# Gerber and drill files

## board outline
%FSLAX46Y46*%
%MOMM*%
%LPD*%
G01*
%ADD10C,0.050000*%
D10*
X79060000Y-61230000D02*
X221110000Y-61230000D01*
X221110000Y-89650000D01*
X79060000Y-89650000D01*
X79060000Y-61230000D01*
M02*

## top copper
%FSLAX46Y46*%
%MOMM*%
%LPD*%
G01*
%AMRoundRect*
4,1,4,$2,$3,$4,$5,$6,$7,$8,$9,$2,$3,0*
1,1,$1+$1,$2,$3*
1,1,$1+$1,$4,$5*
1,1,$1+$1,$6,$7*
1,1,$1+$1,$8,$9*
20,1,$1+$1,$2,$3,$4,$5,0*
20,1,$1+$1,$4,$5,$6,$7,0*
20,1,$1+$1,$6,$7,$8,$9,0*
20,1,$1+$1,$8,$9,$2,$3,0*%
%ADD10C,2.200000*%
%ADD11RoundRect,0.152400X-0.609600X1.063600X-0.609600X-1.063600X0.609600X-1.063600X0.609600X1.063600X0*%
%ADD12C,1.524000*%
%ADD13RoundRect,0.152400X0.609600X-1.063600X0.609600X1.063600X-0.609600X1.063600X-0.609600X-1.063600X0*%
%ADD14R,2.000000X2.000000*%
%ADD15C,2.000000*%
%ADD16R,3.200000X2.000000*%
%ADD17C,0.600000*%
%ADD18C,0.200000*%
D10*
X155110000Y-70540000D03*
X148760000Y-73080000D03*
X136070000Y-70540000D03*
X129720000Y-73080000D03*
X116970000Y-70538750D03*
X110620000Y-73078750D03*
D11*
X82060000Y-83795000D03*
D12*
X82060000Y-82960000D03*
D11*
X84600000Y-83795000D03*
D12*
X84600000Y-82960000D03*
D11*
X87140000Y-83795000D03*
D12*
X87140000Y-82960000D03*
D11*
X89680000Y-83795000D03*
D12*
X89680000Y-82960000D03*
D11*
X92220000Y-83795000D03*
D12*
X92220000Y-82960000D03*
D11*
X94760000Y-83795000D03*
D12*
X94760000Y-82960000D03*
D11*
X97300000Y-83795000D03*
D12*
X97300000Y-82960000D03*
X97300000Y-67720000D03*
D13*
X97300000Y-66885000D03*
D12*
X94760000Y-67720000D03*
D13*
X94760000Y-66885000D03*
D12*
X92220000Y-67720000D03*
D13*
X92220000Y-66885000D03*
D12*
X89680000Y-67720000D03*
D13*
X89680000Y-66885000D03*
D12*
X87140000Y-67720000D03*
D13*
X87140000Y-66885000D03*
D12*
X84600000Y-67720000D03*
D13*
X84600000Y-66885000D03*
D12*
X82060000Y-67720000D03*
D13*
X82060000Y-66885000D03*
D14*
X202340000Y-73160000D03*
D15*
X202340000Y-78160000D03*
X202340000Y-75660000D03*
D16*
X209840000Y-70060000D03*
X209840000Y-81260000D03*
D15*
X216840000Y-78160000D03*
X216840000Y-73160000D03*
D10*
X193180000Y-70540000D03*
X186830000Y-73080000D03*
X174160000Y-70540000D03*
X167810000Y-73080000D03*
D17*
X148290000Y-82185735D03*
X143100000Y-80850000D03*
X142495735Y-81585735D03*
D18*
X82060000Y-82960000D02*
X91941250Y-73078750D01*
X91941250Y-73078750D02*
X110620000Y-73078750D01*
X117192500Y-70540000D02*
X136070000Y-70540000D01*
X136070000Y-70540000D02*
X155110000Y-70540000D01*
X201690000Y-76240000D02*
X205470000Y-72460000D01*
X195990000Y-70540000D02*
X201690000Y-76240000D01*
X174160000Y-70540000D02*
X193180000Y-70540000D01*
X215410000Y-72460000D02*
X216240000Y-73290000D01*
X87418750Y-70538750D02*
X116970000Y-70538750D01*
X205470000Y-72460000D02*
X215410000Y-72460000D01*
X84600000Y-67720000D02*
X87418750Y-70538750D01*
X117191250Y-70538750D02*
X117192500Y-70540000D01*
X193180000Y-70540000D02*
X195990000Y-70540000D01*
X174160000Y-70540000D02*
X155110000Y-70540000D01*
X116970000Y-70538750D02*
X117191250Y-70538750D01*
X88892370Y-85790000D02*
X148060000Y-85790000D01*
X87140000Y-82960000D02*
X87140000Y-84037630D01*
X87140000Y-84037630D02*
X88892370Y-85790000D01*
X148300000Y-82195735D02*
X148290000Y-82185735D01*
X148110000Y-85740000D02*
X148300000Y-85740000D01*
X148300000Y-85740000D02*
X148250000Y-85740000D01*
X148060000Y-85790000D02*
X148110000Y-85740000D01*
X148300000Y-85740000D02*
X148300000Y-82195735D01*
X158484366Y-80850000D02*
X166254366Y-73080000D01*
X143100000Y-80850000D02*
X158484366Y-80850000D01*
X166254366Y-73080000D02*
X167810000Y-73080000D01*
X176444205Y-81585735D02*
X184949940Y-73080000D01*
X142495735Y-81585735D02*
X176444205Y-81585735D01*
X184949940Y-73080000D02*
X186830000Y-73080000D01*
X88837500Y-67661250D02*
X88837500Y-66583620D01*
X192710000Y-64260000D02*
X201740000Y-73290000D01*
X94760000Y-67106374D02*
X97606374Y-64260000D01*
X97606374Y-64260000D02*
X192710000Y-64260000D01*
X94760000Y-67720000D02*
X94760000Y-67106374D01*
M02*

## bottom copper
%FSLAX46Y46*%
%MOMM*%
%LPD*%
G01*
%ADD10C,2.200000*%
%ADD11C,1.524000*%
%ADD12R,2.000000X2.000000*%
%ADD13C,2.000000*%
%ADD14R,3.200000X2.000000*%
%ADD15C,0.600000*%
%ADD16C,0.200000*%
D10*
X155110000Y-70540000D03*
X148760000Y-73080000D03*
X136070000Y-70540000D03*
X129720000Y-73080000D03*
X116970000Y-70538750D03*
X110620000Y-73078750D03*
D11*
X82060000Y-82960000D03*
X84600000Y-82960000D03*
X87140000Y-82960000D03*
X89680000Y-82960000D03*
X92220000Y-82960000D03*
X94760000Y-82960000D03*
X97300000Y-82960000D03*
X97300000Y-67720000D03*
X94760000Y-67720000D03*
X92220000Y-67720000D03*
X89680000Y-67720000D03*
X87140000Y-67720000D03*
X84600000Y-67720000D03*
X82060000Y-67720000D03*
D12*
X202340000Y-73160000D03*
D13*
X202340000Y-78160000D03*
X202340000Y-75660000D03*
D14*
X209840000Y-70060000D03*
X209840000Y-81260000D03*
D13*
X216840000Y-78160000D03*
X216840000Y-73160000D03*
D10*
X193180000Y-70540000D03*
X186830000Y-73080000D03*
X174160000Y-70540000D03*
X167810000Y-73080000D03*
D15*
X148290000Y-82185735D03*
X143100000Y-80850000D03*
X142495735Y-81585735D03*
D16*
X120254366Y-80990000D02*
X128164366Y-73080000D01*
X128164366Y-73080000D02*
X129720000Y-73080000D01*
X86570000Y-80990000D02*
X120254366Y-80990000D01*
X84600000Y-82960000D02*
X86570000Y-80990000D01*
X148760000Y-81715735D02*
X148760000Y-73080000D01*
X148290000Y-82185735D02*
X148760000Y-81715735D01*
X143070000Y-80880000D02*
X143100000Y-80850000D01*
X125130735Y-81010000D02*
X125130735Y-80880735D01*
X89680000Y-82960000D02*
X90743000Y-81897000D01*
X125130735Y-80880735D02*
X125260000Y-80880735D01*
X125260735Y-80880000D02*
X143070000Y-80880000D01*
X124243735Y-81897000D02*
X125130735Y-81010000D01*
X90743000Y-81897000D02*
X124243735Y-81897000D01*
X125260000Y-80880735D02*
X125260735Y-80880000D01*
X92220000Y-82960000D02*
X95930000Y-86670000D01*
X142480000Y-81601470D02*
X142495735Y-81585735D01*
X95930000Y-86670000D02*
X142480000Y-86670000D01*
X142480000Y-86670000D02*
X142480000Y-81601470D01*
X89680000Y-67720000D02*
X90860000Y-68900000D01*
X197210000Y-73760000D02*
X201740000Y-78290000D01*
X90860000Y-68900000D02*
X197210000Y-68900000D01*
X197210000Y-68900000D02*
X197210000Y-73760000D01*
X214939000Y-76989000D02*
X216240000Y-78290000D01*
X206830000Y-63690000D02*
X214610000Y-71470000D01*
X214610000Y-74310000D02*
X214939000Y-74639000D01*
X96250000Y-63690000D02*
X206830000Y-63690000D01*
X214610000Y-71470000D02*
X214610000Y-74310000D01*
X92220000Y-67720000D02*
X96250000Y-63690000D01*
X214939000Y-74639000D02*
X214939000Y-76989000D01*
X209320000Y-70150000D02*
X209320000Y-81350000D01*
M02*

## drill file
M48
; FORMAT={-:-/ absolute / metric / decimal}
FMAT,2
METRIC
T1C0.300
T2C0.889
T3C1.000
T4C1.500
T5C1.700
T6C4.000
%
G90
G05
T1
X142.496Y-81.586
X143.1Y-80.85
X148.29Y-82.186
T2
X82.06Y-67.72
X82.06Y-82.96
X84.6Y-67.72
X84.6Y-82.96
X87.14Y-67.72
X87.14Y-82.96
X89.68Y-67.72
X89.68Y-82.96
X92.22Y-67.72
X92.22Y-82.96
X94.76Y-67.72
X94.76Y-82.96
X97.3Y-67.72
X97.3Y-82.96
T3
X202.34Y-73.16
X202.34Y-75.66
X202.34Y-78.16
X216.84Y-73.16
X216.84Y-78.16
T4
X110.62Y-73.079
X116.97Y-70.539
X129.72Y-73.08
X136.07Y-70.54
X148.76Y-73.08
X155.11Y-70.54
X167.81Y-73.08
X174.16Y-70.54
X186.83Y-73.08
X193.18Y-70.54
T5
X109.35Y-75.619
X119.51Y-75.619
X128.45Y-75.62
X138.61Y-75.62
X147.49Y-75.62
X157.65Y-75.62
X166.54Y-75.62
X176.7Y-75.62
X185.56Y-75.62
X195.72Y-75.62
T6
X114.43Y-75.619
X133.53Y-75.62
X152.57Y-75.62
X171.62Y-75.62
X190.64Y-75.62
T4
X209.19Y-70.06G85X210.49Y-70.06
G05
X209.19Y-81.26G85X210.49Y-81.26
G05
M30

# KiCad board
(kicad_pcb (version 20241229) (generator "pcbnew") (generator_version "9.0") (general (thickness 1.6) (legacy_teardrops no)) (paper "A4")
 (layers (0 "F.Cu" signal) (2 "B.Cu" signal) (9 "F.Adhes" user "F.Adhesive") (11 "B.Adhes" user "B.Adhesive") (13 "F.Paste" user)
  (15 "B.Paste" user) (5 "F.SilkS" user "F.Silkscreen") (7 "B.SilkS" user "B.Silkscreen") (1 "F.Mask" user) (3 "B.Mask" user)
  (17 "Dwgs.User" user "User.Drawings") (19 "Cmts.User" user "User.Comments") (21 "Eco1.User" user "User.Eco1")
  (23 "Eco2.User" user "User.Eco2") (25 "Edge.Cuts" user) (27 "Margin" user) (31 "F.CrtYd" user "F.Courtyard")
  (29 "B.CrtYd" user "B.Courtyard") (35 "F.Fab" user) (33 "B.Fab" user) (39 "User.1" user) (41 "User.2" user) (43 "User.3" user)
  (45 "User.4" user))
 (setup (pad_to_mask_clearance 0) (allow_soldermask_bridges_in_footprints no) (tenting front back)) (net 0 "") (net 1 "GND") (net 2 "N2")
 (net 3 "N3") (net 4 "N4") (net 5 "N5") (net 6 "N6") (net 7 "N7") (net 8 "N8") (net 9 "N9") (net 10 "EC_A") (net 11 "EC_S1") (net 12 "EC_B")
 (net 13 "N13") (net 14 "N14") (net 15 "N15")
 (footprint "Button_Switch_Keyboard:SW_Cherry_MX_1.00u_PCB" (layer "F.Cu") (at 155.11 70.54)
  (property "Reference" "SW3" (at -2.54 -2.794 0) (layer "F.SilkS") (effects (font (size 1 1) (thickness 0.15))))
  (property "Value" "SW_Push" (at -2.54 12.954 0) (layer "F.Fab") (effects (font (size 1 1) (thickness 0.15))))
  (pad "" np_thru_hole circle (at -7.62 5.08) (size 1.7 1.7) (drill 1.7) (layers "*.Cu" "*.Mask"))
  (pad "" np_thru_hole circle (at -2.54 5.08) (size 4 4) (drill 4) (layers "*.Cu" "*.Mask"))
  (pad "" np_thru_hole circle (at 2.54 5.08) (size 1.7 1.7) (drill 1.7) (layers "*.Cu" "*.Mask"))
  (pad "1" thru_hole circle (at 0 0) (size 2.2 2.2) (drill 1.5) (layers "*.Cu" "*.Mask") (remove_unused_layers no) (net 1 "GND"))
  (pad "2" thru_hole circle (at -6.35 2.54) (size 2.2 2.2) (drill 1.5) (layers "*.Cu" "*.Mask") (remove_unused_layers no) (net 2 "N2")))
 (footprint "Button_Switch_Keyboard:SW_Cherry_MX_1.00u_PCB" (layer "F.Cu") (at 136.07 70.54)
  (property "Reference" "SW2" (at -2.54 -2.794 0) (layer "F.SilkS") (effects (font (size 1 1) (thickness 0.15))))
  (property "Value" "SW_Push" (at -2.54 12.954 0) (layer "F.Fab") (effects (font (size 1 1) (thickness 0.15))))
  (pad "" np_thru_hole circle (at -7.62 5.08) (size 1.7 1.7) (drill 1.7) (layers "*.Cu" "*.Mask"))
  (pad "" np_thru_hole circle (at -2.54 5.08) (size 4 4) (drill 4) (layers "*.Cu" "*.Mask"))
  (pad "" np_thru_hole circle (at 2.54 5.08) (size 1.7 1.7) (drill 1.7) (layers "*.Cu" "*.Mask"))
  (pad "1" thru_hole circle (at 0 0) (size 2.2 2.2) (drill 1.5) (layers "*.Cu" "*.Mask") (remove_unused_layers no) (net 1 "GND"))
  (pad "2" thru_hole circle (at -6.35 2.54) (size 2.2 2.2) (drill 1.5) (layers "*.Cu" "*.Mask") (remove_unused_layers no) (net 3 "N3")))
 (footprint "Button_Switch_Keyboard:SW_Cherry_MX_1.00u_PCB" (layer "F.Cu") (at 116.97 70.53875)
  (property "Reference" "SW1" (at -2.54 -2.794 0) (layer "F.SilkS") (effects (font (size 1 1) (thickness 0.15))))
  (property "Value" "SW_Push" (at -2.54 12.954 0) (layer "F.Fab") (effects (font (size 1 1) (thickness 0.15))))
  (pad "" np_thru_hole circle (at -7.62 5.08) (size 1.7 1.7) (drill 1.7) (layers "*.Cu" "*.Mask"))
  (pad "" np_thru_hole circle (at -2.54 5.08) (size 4 4) (drill 4) (layers "*.Cu" "*.Mask"))
  (pad "" np_thru_hole circle (at 2.54 5.08) (size 1.7 1.7) (drill 1.7) (layers "*.Cu" "*.Mask"))
  (pad "1" thru_hole circle (at 0 0) (size 2.2 2.2) (drill 1.5) (layers "*.Cu" "*.Mask") (remove_unused_layers no) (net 1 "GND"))
  (pad "2" thru_hole circle (at -6.35 2.54) (size 2.2 2.2) (drill 1.5) (layers "*.Cu" "*.Mask") (remove_unused_layers no) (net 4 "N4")))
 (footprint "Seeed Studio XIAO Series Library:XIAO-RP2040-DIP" (layer "F.Cu") (at 89.68 75.34 90)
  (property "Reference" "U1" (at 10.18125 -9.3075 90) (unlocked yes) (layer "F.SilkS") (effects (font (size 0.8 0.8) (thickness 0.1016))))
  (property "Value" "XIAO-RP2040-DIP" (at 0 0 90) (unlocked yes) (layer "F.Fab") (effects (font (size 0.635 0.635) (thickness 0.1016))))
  (pad "1" smd roundrect (at -8.455 -7.62 270) (size 2.432 1.524) (layers "F.Cu" "F.Mask") (roundrect_rratio 0.1) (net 4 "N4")
   (thermal_bridge_angle 45))
  (pad "1" thru_hole circle (at -7.62 -7.62 270) (size 1.524 1.524) (drill 0.889) (layers "*.Cu" "*.Mask") (remove_unused_layers no)
   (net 4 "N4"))
  (pad "2" smd roundrect (at -8.455 -5.08 270) (size 2.432 1.524) (layers "F.Cu" "F.Mask") (roundrect_rratio 0.1) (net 3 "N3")
   (thermal_bridge_angle 45))
  (pad "2" thru_hole circle (at -7.62 -5.08 270) (size 1.524 1.524) (drill 0.889) (layers "*.Cu" "*.Mask") (remove_unused_layers no)
   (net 3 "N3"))
  (pad "3" smd roundrect (at -8.455 -2.54 270) (size 2.432 1.524) (layers "F.Cu" "F.Mask") (roundrect_rratio 0.1) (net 2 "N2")
   (thermal_bridge_angle 45))
  (pad "3" thru_hole circle (at -7.62 -2.54 270) (size 1.524 1.524) (drill 0.889) (layers "*.Cu" "*.Mask") (remove_unused_layers no)
   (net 2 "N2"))
  (pad "4" smd roundrect (at -8.455 0 270) (size 2.432 1.524) (layers "F.Cu" "F.Mask") (roundrect_rratio 0.1) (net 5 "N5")
   (thermal_bridge_angle 45))
  (pad "4" thru_hole circle (at -7.62 0 270) (size 1.524 1.524) (drill 0.889) (layers "*.Cu" "*.Mask") (remove_unused_layers no)
   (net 5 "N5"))
  (pad "5" smd roundrect (at -8.455 2.54 270) (size 2.432 1.524) (layers "F.Cu" "F.Mask") (roundrect_rratio 0.1) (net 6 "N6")
   (thermal_bridge_angle 45))
  (pad "5" thru_hole circle (at -7.62 2.54 270) (size 1.524 1.524) (drill 0.889) (layers "*.Cu" "*.Mask") (remove_unused_layers no)
   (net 6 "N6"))
  (pad "6" smd roundrect (at -8.455 5.08 270) (size 2.432 1.524) (layers "F.Cu" "F.Mask") (roundrect_rratio 0.1) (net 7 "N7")
   (thermal_bridge_angle 45))
  (pad "6" thru_hole circle (at -7.62 5.08 270) (size 1.524 1.524) (drill 0.889) (layers "*.Cu" "*.Mask") (remove_unused_layers no)
   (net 7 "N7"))
  (pad "7" smd roundrect (at -8.455 7.62 270) (size 2.432 1.524) (layers "F.Cu" "F.Mask") (roundrect_rratio 0.1) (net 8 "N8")
   (thermal_bridge_angle 45))
  (pad "7" thru_hole circle (at -7.62 7.62 270) (size 1.524 1.524) (drill 0.889) (layers "*.Cu" "*.Mask") (remove_unused_layers no)
   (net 8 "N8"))
  (pad "8" thru_hole circle (at 7.62 7.62 90) (size 1.524 1.524) (drill 0.889) (layers "*.Cu" "*.Mask") (remove_unused_layers no)
   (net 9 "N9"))
  (pad "8" smd roundrect (at 8.455 7.62 90) (size 2.432 1.524) (layers "F.Cu" "F.Mask") (roundrect_rratio 0.1) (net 9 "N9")
   (thermal_bridge_angle 45))
  (pad "9" thru_hole circle (at 7.62 5.08 90) (size 1.524 1.524) (drill 0.889) (layers "*.Cu" "*.Mask") (remove_unused_layers no)
   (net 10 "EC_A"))
  (pad "9" smd roundrect (at 8.455 5.08 90) (size 2.432 1.524) (layers "F.Cu" "F.Mask") (roundrect_rratio 0.1) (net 10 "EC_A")
   (thermal_bridge_angle 45))
  (pad "10" thru_hole circle (at 7.62 2.54 90) (size 1.524 1.524) (drill 0.889) (layers "*.Cu" "*.Mask") (remove_unused_layers no)
   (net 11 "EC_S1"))
  (pad "10" smd roundrect (at 8.455 2.54 90) (size 2.432 1.524) (layers "F.Cu" "F.Mask") (roundrect_rratio 0.1) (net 11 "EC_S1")
   (thermal_bridge_angle 45))
  (pad "11" thru_hole circle (at 7.62 0 90) (size 1.524 1.524) (drill 0.889) (layers "*.Cu" "*.Mask") (remove_unused_layers no)
   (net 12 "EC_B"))
  (pad "11" smd roundrect (at 8.455 0 90) (size 2.432 1.524) (layers "F.Cu" "F.Mask") (roundrect_rratio 0.1) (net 12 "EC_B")
   (thermal_bridge_angle 45))
  (pad "12" thru_hole circle (at 7.62 -2.54 90) (size 1.524 1.524) (drill 0.889) (layers "*.Cu" "*.Mask") (remove_unused_layers no)
   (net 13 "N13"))
  (pad "12" smd roundrect (at 8.455 -2.54 90) (size 2.432 1.524) (layers "F.Cu" "F.Mask") (roundrect_rratio 0.1) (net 13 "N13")
   (thermal_bridge_angle 45))
  (pad "13" thru_hole circle (at 7.62 -5.08 90) (size 1.524 1.524) (drill 0.889) (layers "*.Cu" "*.Mask") (remove_unused_layers no)
   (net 1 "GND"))
  (pad "13" smd roundrect (at 8.455 -5.08 90) (size 2.432 1.524) (layers "F.Cu" "F.Mask") (roundrect_rratio 0.1) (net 1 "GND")
   (thermal_bridge_angle 45))
  (pad "14" thru_hole circle (at 7.62 -7.62 90) (size 1.524 1.524) (drill 0.889) (layers "*.Cu" "*.Mask") (remove_unused_layers no)
   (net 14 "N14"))
  (pad "14" smd roundrect (at 8.455 -7.62 90) (size 2.432 1.524) (layers "F.Cu" "F.Mask") (roundrect_rratio 0.1) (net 14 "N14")
   (thermal_bridge_angle 45)))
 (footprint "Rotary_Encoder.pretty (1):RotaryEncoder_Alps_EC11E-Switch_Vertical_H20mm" (layer "F.Cu") (at 202.34 73.16)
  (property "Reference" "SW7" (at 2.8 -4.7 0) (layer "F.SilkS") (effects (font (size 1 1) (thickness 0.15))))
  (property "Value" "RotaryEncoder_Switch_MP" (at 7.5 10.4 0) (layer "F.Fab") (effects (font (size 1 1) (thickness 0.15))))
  (pad "A" thru_hole rect (at 0 0) (size 2 2) (drill 1) (layers "*.Cu" "*.Mask") (remove_unused_layers no) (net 10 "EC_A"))
  (pad "B" thru_hole circle (at 0 5) (size 2 2) (drill 1) (layers "*.Cu" "*.Mask") (remove_unused_layers no) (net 12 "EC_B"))
  (pad "C" thru_hole circle (at 0 2.5) (size 2 2) (drill 1) (layers "*.Cu" "*.Mask") (remove_unused_layers no) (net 1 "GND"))
  (pad "MP" thru_hole rect (at 7.5 -3.1) (size 3.2 2) (drill oval 2.8 1.5) (layers "*.Cu" "*.Mask") (remove_unused_layers no) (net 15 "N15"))
  (pad "MP" thru_hole rect (at 7.5 8.1) (size 3.2 2) (drill oval 2.8 1.5) (layers "*.Cu" "*.Mask") (remove_unused_layers no) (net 15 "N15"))
  (pad "S1" thru_hole circle (at 14.5 5) (size 2 2) (drill 1) (layers "*.Cu" "*.Mask") (remove_unused_layers no) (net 11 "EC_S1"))
  (pad "S2" thru_hole circle (at 14.5 0) (size 2 2) (drill 1) (layers "*.Cu" "*.Mask") (remove_unused_layers no) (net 1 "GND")))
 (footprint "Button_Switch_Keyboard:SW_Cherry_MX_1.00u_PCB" (layer "F.Cu") (at 193.18 70.54)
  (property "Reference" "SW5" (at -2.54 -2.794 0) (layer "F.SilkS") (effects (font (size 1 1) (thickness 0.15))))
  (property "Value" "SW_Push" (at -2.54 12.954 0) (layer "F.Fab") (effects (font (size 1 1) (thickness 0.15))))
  (pad "" np_thru_hole circle (at -7.62 5.08) (size 1.7 1.7) (drill 1.7) (layers "*.Cu" "*.Mask"))
  (pad "" np_thru_hole circle (at -2.54 5.08) (size 4 4) (drill 4) (layers "*.Cu" "*.Mask"))
  (pad "" np_thru_hole circle (at 2.54 5.08) (size 1.7 1.7) (drill 1.7) (layers "*.Cu" "*.Mask"))
  (pad "1" thru_hole circle (at 0 0) (size 2.2 2.2) (drill 1.5) (layers "*.Cu" "*.Mask") (remove_unused_layers no) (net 1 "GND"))
  (pad "2" thru_hole circle (at -6.35 2.54) (size 2.2 2.2) (drill 1.5) (layers "*.Cu" "*.Mask") (remove_unused_layers no) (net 6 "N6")))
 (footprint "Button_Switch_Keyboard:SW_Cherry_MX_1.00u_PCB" (layer "F.Cu") (at 174.16 70.54)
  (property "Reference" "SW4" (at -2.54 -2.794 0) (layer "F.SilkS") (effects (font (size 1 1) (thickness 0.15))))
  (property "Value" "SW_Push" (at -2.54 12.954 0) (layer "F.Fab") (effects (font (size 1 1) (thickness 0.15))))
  (pad "" np_thru_hole circle (at -7.62 5.08) (size 1.7 1.7) (drill 1.7) (layers "*.Cu" "*.Mask"))
  (pad "" np_thru_hole circle (at -2.54 5.08) (size 4 4) (drill 4) (layers "*.Cu" "*.Mask"))
  (pad "" np_thru_hole circle (at 2.54 5.08) (size 1.7 1.7) (drill 1.7) (layers "*.Cu" "*.Mask"))
  (pad "1" thru_hole circle (at 0 0) (size 2.2 2.2) (drill 1.5) (layers "*.Cu" "*.Mask") (remove_unused_layers no) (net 1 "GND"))
  (pad "2" thru_hole circle (at -6.35 2.54) (size 2.2 2.2) (drill 1.5) (layers "*.Cu" "*.Mask") (remove_unused_layers no) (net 5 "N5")))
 (gr_rect (start 79.06 61.23) (end 221.11 89.65) (stroke (width 0.05) (type default)) (fill no) (layer "Edge.Cuts"))
 (segment (start 82.06 82.96) (end 91.94125 73.07875) (width 0.2) (layer "F.Cu") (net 4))
 (segment (start 91.94125 73.07875) (end 110.62 73.07875) (width 0.2) (layer "F.Cu") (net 4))
 (segment (start 117.1925 70.54) (end 136.07 70.54) (width 0.2) (layer "F.Cu") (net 1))
 (segment (start 136.07 70.54) (end 155.11 70.54) (width 0.2) (layer "F.Cu") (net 1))
 (segment (start 201.69 76.24) (end 205.47 72.46) (width 0.2) (layer "F.Cu") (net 1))
 (segment (start 195.99 70.54) (end 201.69 76.24) (width 0.2) (layer "F.Cu") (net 1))
 (segment (start 174.16 70.54) (end 193.18 70.54) (width 0.2) (layer "F.Cu") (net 1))
 (segment (start 215.41 72.46) (end 216.24 73.29) (width 0.2) (layer "F.Cu") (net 1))
 (segment (start 87.41875 70.53875) (end 116.97 70.53875) (width 0.2) (layer "F.Cu") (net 1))
 (segment (start 205.47 72.46) (end 215.41 72.46) (width 0.2) (layer "F.Cu") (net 1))
 (segment (start 84.6 67.72) (end 87.41875 70.53875) (width 0.2) (layer "F.Cu") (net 1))
 (segment (start 117.19125 70.53875) (end 117.1925 70.54) (width 0.2) (layer "F.Cu") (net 1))
 (segment (start 193.18 70.54) (end 195.99 70.54) (width 0.2) (layer "F.Cu") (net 1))
 (segment (start 174.16 70.54) (end 155.11 70.54) (width 0.2) (layer "F.Cu") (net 1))
 (segment (start 116.97 70.53875) (end 117.19125 70.53875) (width 0.2) (layer "F.Cu") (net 1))
 (segment (start 120.254366 80.99) (end 128.164366 73.08) (width 0.2) (layer "B.Cu") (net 3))
 (segment (start 128.164366 73.08) (end 129.72 73.08) (width 0.2) (layer "B.Cu") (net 3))
 (segment (start 86.57 80.99) (end 120.254366 80.99) (width 0.2) (layer "B.Cu") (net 3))
 (segment (start 84.6 82.96) (end 86.57 80.99) (width 0.2) (layer "B.Cu") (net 3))
 (segment (start 88.89237 85.79) (end 148.06 85.79) (width 0.2) (layer "F.Cu") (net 2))
 (segment (start 87.14 82.96) (end 87.14 84.03763) (width 0.2) (layer "F.Cu") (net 2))
 (segment (start 87.14 84.03763) (end 88.89237 85.79) (width 0.2) (layer "F.Cu") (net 2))
 (segment (start 148.3 82.195735) (end 148.29 82.185735) (width 0.2) (layer "F.Cu") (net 2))
 (segment (start 148.11 85.74) (end 148.3 85.74) (width 0.2) (layer "F.Cu") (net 2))
 (segment (start 148.3 85.74) (end 148.25 85.74) (width 0.2) (layer "F.Cu") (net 2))
 (segment (start 148.06 85.79) (end 148.11 85.74) (width 0.2) (layer "F.Cu") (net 2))
 (segment (start 148.3 85.74) (end 148.3 82.195735) (width 0.2) (layer "F.Cu") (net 2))
 (via (at 148.29 82.185735) (size 0.6) (drill 0.3) (layers "F.Cu" "B.Cu") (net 2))
 (segment (start 148.76 81.715735) (end 148.76 73.08) (width 0.2) (layer "B.Cu") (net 2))
 (segment (start 148.29 82.185735) (end 148.76 81.715735) (width 0.2) (layer "B.Cu") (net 2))
 (segment (start 158.484366 80.85) (end 166.254366 73.08) (width 0.2) (layer "F.Cu") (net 5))
 (segment (start 143.1 80.85) (end 158.484366 80.85) (width 0.2) (layer "F.Cu") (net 5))
 (segment (start 166.254366 73.08) (end 167.81 73.08) (width 0.2) (layer "F.Cu") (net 5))
 (via (at 143.1 80.85) (size 0.6) (drill 0.3) (layers "F.Cu" "B.Cu") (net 5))
 (segment (start 143.07 80.88) (end 143.1 80.85) (width 0.2) (layer "B.Cu") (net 5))
 (segment (start 125.130735 81.01) (end 125.130735 80.880735) (width 0.2) (layer "B.Cu") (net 5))
 (segment (start 89.68 82.96) (end 90.743 81.897) (width 0.2) (layer "B.Cu") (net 5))
 (segment (start 125.130735 80.880735) (end 125.26 80.880735) (width 0.2) (layer "B.Cu") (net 5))
 (segment (start 125.260735 80.88) (end 143.07 80.88) (width 0.2) (layer "B.Cu") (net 5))
 (segment (start 124.243735 81.897) (end 125.130735 81.01) (width 0.2) (layer "B.Cu") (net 5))
 (segment (start 90.743 81.897) (end 124.243735 81.897) (width 0.2) (layer "B.Cu") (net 5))
 (segment (start 125.26 80.880735) (end 125.260735 80.88) (width 0.2) (layer "B.Cu") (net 5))
 (segment (start 176.444205 81.585735) (end 184.94994 73.08) (width 0.2) (layer "F.Cu") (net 6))
 (segment (start 142.495735 81.585735) (end 176.444205 81.585735) (width 0.2) (layer "F.Cu") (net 6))
 (segment (start 184.94994 73.08) (end 186.83 73.08) (width 0.2) (layer "F.Cu") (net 6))
 (via (at 142.495735 81.585735) (size 0.6) (drill 0.3) (layers "F.Cu" "B.Cu") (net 6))
 (segment (start 92.22 82.96) (end 95.93 86.67) (width 0.2) (layer "B.Cu") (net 6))
 (segment (start 142.48 81.60147) (end 142.495735 81.585735) (width 0.2) (layer "B.Cu") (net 6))
 (segment (start 95.93 86.67) (end 142.48 86.67) (width 0.2) (layer "B.Cu") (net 6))
 (segment (start 142.48 86.67) (end 142.48 81.60147) (width 0.2) (layer "B.Cu") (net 6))
 (segment (start 88.8375 67.66125) (end 88.8375 66.58362) (width 0.2) (layer "F.Cu") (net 12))
 (segment (start 89.68 67.72) (end 90.86 68.9) (width 0.2) (layer "B.Cu") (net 12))
 (segment (start 197.21 73.76) (end 201.74 78.29) (width 0.2) (layer "B.Cu") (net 12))
 (segment (start 90.86 68.9) (end 197.21 68.9) (width 0.2) (layer "B.Cu") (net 12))
 (segment (start 197.21 68.9) (end 197.21 73.76) (width 0.2) (layer "B.Cu") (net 12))
 (segment (start 192.71 64.26) (end 201.74 73.29) (width 0.2) (layer "F.Cu") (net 10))
 (segment (start 94.76 67.106374) (end 97.606374 64.26) (width 0.2) (layer "F.Cu") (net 10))
 (segment (start 97.606374 64.26) (end 192.71 64.26) (width 0.2) (layer "F.Cu") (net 10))
 (segment (start 94.76 67.72) (end 94.76 67.106374) (width 0.2) (layer "F.Cu") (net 10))
 (segment (start 214.939 76.989) (end 216.24 78.29) (width 0.2) (layer "B.Cu") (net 11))
 (segment (start 206.83 63.69) (end 214.61 71.47) (width 0.2) (layer "B.Cu") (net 11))
 (segment (start 214.61 74.31) (end 214.939 74.639) (width 0.2) (layer "B.Cu") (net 11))
 (segment (start 96.25 63.69) (end 206.83 63.69) (width 0.2) (layer "B.Cu") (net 11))
 (segment (start 214.61 71.47) (end 214.61 74.31) (width 0.2) (layer "B.Cu") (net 11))
 (segment (start 92.22 67.72) (end 96.25 63.69) (width 0.2) (layer "B.Cu") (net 11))
 (segment (start 214.939 74.639) (end 214.939 76.989) (width 0.2) (layer "B.Cu") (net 11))
 (segment (start 209.32 70.15) (end 209.32 81.35) (width 0.2) (layer "B.Cu") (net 15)))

